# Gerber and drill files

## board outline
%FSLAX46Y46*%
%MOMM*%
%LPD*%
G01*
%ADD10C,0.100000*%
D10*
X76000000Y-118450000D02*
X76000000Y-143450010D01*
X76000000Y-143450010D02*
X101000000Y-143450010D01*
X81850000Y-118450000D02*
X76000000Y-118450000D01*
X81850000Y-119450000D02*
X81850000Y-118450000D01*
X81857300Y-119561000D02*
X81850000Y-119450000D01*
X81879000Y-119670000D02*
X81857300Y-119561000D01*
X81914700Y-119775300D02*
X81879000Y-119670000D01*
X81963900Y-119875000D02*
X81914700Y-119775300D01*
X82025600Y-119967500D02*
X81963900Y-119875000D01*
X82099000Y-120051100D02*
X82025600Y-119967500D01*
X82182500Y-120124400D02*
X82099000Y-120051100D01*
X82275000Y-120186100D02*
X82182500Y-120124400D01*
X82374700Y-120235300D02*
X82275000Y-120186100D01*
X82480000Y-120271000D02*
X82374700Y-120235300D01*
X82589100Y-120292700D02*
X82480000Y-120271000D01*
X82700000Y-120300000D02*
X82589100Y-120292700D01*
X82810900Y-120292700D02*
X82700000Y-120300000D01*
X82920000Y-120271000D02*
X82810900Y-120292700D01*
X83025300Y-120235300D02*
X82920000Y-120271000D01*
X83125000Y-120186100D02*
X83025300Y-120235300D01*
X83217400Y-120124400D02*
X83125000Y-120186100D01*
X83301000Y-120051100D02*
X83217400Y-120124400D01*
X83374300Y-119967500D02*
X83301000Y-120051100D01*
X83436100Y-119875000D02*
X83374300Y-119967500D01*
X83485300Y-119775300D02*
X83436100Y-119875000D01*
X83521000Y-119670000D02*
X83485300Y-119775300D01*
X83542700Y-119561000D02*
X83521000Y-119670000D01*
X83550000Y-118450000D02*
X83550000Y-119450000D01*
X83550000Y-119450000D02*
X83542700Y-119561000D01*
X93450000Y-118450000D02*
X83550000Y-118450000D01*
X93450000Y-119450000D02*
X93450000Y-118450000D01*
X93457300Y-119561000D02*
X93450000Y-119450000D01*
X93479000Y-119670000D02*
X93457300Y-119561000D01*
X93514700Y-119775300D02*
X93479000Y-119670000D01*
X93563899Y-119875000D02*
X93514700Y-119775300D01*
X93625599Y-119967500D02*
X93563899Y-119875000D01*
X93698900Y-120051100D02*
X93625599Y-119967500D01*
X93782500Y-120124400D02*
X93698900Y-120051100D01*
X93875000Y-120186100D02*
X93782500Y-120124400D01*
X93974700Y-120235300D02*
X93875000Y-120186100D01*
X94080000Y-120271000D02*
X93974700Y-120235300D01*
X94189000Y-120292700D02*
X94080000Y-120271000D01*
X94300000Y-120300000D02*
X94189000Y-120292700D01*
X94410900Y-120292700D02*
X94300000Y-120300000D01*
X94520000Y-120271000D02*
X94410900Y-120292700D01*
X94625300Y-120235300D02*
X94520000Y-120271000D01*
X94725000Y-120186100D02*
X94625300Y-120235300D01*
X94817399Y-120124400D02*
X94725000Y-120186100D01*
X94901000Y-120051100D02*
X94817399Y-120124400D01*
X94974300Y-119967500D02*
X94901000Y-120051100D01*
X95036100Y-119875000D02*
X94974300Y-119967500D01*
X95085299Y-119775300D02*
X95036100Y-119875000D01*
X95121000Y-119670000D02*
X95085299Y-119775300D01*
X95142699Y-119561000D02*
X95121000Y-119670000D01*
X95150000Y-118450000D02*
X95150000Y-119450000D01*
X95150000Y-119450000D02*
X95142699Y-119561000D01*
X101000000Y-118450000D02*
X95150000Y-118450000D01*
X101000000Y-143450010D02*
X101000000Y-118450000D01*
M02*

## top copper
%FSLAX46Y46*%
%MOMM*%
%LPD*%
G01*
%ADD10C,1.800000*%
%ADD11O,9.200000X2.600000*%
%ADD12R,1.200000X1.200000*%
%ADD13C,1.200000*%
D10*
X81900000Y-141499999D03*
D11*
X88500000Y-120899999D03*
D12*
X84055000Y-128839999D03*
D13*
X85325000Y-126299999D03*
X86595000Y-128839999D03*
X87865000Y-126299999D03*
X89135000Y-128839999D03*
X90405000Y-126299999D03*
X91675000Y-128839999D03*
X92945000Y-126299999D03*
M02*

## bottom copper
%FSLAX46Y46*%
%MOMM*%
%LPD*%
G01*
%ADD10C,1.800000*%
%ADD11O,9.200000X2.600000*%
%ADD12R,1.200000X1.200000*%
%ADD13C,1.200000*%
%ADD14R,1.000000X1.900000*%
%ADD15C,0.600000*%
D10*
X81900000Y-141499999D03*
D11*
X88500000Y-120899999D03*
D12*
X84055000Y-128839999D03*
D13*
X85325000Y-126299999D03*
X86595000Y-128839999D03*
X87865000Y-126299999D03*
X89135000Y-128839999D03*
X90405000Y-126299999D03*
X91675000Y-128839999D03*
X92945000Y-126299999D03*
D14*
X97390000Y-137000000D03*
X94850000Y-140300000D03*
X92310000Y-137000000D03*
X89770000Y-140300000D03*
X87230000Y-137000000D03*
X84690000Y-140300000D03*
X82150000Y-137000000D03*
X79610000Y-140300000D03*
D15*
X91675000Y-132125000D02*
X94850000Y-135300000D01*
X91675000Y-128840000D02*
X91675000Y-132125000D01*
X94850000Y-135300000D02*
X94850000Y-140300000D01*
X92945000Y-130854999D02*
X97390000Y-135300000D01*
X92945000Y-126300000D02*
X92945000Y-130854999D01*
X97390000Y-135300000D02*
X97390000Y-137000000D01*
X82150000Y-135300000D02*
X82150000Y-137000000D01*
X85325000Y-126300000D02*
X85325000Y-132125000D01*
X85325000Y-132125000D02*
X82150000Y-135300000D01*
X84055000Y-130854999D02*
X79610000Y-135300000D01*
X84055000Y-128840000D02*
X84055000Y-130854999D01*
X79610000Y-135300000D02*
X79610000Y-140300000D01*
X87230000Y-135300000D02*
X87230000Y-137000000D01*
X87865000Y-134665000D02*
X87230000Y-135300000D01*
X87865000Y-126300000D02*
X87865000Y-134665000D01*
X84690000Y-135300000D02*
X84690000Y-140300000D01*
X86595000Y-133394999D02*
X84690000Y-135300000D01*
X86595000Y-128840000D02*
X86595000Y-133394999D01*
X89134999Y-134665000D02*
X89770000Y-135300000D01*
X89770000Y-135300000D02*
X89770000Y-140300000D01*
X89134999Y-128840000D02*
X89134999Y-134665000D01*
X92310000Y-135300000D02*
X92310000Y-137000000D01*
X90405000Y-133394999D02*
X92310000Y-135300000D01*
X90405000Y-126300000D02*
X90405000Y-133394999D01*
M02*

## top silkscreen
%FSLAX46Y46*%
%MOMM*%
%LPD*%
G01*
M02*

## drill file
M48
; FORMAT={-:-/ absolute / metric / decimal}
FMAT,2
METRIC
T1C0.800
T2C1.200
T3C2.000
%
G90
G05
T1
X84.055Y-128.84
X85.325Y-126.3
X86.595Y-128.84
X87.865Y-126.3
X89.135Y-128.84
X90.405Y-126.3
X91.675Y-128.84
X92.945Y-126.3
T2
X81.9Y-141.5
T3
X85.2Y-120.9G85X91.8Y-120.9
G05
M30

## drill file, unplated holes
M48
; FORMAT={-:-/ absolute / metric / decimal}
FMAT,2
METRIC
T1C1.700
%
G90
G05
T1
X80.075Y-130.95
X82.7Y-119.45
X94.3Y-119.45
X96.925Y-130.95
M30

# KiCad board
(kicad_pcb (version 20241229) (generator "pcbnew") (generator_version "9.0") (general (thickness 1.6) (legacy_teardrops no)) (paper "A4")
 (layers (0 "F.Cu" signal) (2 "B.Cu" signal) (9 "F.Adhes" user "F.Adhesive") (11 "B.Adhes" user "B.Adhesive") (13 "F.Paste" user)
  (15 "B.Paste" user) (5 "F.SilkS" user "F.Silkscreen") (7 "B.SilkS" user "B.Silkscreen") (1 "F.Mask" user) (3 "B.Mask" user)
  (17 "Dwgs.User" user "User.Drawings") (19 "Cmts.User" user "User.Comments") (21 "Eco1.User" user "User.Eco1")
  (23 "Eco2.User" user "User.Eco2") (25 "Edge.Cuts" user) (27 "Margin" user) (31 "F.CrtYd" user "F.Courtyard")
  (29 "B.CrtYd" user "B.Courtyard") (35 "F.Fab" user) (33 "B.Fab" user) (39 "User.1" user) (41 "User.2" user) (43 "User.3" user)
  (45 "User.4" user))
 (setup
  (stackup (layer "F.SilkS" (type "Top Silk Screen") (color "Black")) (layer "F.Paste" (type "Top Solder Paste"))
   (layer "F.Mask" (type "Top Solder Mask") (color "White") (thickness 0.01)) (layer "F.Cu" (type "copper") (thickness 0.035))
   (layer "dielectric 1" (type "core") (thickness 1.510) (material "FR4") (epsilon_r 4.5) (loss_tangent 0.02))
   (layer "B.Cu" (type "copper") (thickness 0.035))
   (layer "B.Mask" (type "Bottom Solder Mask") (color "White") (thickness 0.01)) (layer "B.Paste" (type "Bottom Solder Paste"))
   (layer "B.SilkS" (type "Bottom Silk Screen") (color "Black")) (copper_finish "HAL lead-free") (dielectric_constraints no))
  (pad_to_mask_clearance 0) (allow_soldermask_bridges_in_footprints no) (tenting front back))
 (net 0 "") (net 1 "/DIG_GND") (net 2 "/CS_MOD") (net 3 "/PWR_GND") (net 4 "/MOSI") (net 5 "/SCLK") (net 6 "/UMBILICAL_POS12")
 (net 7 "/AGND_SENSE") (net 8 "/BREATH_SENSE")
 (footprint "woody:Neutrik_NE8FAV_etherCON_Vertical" (layer "F.Cu") (at 88.5 130.949999)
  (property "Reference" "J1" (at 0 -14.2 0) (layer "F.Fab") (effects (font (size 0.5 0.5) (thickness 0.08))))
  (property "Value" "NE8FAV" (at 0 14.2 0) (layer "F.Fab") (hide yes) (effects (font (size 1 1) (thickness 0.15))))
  (pad "" np_thru_hole circle (at -8.425 0) (size 1.7 1.7) (drill 1.7) (layers "*.Cu" "*.Mask"))
  (pad "" thru_hole circle (at -6.6 10.55) (size 1.8 1.8) (drill 1.2) (layers "*.Cu" "*.Mask") (remove_unused_layers no))
  (pad "" np_thru_hole circle (at -5.8 -11.5) (size 1.7 1.7) (drill 1.7) (layers "*.Cu" "*.Mask"))
  (pad "" thru_hole oval (at 0 -10.05) (size 9.2 2.6) (drill oval 8.6 2) (layers "*.Cu" "*.Mask") (remove_unused_layers no))
  (pad "" np_thru_hole circle (at 5.8 -11.5) (size 1.7 1.7) (drill 1.7) (layers "*.Cu" "*.Mask"))
  (pad "" np_thru_hole circle (at 8.425 0) (size 1.7 1.7) (drill 1.7) (layers "*.Cu" "*.Mask"))
  (pad "1" thru_hole rect (at -4.445 -2.11) (size 1.2 1.2) (drill 0.8) (layers "*.Cu" "*.Mask") (remove_unused_layers no) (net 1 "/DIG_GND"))
  (pad "2" thru_hole circle (at -3.175 -4.65) (size 1.2 1.2) (drill 0.8) (layers "*.Cu" "*.Mask") (remove_unused_layers no)
   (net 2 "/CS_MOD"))
  (pad "3" thru_hole circle (at -1.905 -2.11) (size 1.2 1.2) (drill 0.8) (layers "*.Cu" "*.Mask") (remove_unused_layers no)
   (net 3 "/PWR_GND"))
  (pad "4" thru_hole circle (at -0.635 -4.65) (size 1.2 1.2) (drill 0.8) (layers "*.Cu" "*.Mask") (remove_unused_layers no) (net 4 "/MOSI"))
  (pad "5" thru_hole circle (at 0.635 -2.11) (size 1.2 1.2) (drill 0.8) (layers "*.Cu" "*.Mask") (remove_unused_layers no) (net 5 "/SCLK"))
  (pad "6" thru_hole circle (at 1.905 -4.65) (size 1.2 1.2) (drill 0.8) (layers "*.Cu" "*.Mask") (remove_unused_layers no)
   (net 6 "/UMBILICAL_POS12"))
  (pad "7" thru_hole circle (at 3.175 -2.11) (size 1.2 1.2) (drill 0.8) (layers "*.Cu" "*.Mask") (remove_unused_layers no)
   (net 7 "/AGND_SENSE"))
  (pad "8" thru_hole circle (at 4.445 -4.65) (size 1.2 1.2) (drill 0.8) (layers "*.Cu" "*.Mask") (remove_unused_layers no)
   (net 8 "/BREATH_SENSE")))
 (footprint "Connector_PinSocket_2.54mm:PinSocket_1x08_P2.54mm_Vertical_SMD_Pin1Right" (layer "B.Cu") (at 88.5 138.65 90)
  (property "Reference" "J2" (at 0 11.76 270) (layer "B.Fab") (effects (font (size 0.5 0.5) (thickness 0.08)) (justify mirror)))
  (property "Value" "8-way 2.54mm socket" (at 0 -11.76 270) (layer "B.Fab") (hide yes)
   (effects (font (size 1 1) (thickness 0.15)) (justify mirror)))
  (pad "1" smd rect (at 1.65 8.89 90) (size 1.9 1) (layers "B.Cu" "B.Mask" "B.Paste") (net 8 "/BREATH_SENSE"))
  (pad "2" smd rect (at -1.65 6.35 90) (size 1.9 1) (layers "B.Cu" "B.Mask" "B.Paste") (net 7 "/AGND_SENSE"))
  (pad "3" smd rect (at 1.65 3.81 90) (size 1.9 1) (layers "B.Cu" "B.Mask" "B.Paste") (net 6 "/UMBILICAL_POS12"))
  (pad "4" smd rect (at -1.65 1.27 90) (size 1.9 1) (layers "B.Cu" "B.Mask" "B.Paste") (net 5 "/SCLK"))
  (pad "5" smd rect (at 1.65 -1.27 90) (size 1.9 1) (layers "B.Cu" "B.Mask" "B.Paste") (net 4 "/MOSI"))
  (pad "6" smd rect (at -1.65 -3.81 90) (size 1.9 1) (layers "B.Cu" "B.Mask" "B.Paste") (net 3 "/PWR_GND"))
  (pad "7" smd rect (at 1.65 -6.35 90) (size 1.9 1) (layers "B.Cu" "B.Mask" "B.Paste") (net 2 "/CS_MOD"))
  (pad "8" smd rect (at -1.65 -8.89 90) (size 1.9 1) (layers "B.Cu" "B.Mask" "B.Paste") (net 1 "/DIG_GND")))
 (gr_line (start 76 118.45) (end 76 143.45001) (stroke (width 0.1) (type default)) (layer "Edge.Cuts"))
 (gr_line (start 76 143.45001) (end 101 143.45001) (stroke (width 0.1) (type default)) (layer "Edge.Cuts"))
 (gr_line (start 81.85 118.45) (end 76 118.45) (stroke (width 0.1) (type default)) (layer "Edge.Cuts"))
 (gr_line (start 81.85 119.45) (end 81.85 118.45) (stroke (width 0.1) (type default)) (layer "Edge.Cuts"))
 (gr_line (start 81.8573 119.561) (end 81.85 119.45) (stroke (width 0.1) (type default)) (layer "Edge.Cuts"))
 (gr_line (start 81.879 119.67) (end 81.8573 119.561) (stroke (width 0.1) (type default)) (layer "Edge.Cuts"))
 (gr_line (start 81.9147 119.7753) (end 81.879 119.67) (stroke (width 0.1) (type default)) (layer "Edge.Cuts"))
 (gr_line (start 81.9639 119.875) (end 81.9147 119.7753) (stroke (width 0.1) (type default)) (layer "Edge.Cuts"))
 (gr_line (start 82.0256 119.9675) (end 81.9639 119.875) (stroke (width 0.1) (type default)) (layer "Edge.Cuts"))
 (gr_line (start 82.099 120.0511) (end 82.0256 119.9675) (stroke (width 0.1) (type default)) (layer "Edge.Cuts"))
 (gr_line (start 82.1825 120.1244) (end 82.099 120.0511) (stroke (width 0.1) (type default)) (layer "Edge.Cuts"))
 (gr_line (start 82.275 120.1861) (end 82.1825 120.1244) (stroke (width 0.1) (type default)) (layer "Edge.Cuts"))
 (gr_line (start 82.3747 120.2353) (end 82.275 120.1861) (stroke (width 0.1) (type default)) (layer "Edge.Cuts"))
 (gr_line (start 82.48 120.271) (end 82.3747 120.2353) (stroke (width 0.1) (type default)) (layer "Edge.Cuts"))
 (gr_line (start 82.5891 120.2927) (end 82.48 120.271) (stroke (width 0.1) (type default)) (layer "Edge.Cuts"))
 (gr_line (start 82.7 120.3) (end 82.5891 120.2927) (stroke (width 0.1) (type default)) (layer "Edge.Cuts"))
 (gr_line (start 82.8109 120.2927) (end 82.7 120.3) (stroke (width 0.1) (type default)) (layer "Edge.Cuts"))
 (gr_line (start 82.92 120.271) (end 82.8109 120.2927) (stroke (width 0.1) (type default)) (layer "Edge.Cuts"))
 (gr_line (start 83.0253 120.2353) (end 82.92 120.271) (stroke (width 0.1) (type default)) (layer "Edge.Cuts"))
 (gr_line (start 83.125 120.1861) (end 83.0253 120.2353) (stroke (width 0.1) (type default)) (layer "Edge.Cuts"))
 (gr_line (start 83.2174 120.1244) (end 83.125 120.1861) (stroke (width 0.1) (type default)) (layer "Edge.Cuts"))
 (gr_line (start 83.301 120.0511) (end 83.2174 120.1244) (stroke (width 0.1) (type default)) (layer "Edge.Cuts"))
 (gr_line (start 83.3743 119.9675) (end 83.301 120.0511) (stroke (width 0.1) (type default)) (layer "Edge.Cuts"))
 (gr_line (start 83.4361 119.875) (end 83.3743 119.9675) (stroke (width 0.1) (type default)) (layer "Edge.Cuts"))
 (gr_line (start 83.4853 119.7753) (end 83.4361 119.875) (stroke (width 0.1) (type default)) (layer "Edge.Cuts"))
 (gr_line (start 83.521 119.67) (end 83.4853 119.7753) (stroke (width 0.1) (type default)) (layer "Edge.Cuts"))
 (gr_line (start 83.5427 119.561) (end 83.521 119.67) (stroke (width 0.1) (type default)) (layer "Edge.Cuts"))
 (gr_line (start 83.55 118.45) (end 83.55 119.45) (stroke (width 0.1) (type default)) (layer "Edge.Cuts"))
 (gr_line (start 83.55 119.45) (end 83.5427 119.561) (stroke (width 0.1) (type default)) (layer "Edge.Cuts"))
 (gr_line (start 93.45 118.45) (end 83.55 118.45) (stroke (width 0.1) (type default)) (layer "Edge.Cuts"))
 (gr_line (start 93.45 119.45) (end 93.45 118.45) (stroke (width 0.1) (type default)) (layer "Edge.Cuts"))
 (gr_line (start 93.4573 119.561) (end 93.45 119.45) (stroke (width 0.1) (type default)) (layer "Edge.Cuts"))
 (gr_line (start 93.479 119.67) (end 93.4573 119.561) (stroke (width 0.1) (type default)) (layer "Edge.Cuts"))
 (gr_line (start 93.5147 119.7753) (end 93.479 119.67) (stroke (width 0.1) (type default)) (layer "Edge.Cuts"))
 (gr_line (start 93.563899 119.875) (end 93.5147 119.7753) (stroke (width 0.1) (type default)) (layer "Edge.Cuts"))
 (gr_line (start 93.625599 119.9675) (end 93.563899 119.875) (stroke (width 0.1) (type default)) (layer "Edge.Cuts"))
 (gr_line (start 93.6989 120.0511) (end 93.625599 119.9675) (stroke (width 0.1) (type default)) (layer "Edge.Cuts"))
 (gr_line (start 93.7825 120.1244) (end 93.6989 120.0511) (stroke (width 0.1) (type default)) (layer "Edge.Cuts"))
 (gr_line (start 93.875 120.1861) (end 93.7825 120.1244) (stroke (width 0.1) (type default)) (layer "Edge.Cuts"))
 (gr_line (start 93.9747 120.2353) (end 93.875 120.1861) (stroke (width 0.1) (type default)) (layer "Edge.Cuts"))
 (gr_line (start 94.08 120.271) (end 93.9747 120.2353) (stroke (width 0.1) (type default)) (layer "Edge.Cuts"))
 (gr_line (start 94.189 120.2927) (end 94.08 120.271) (stroke (width 0.1) (type default)) (layer "Edge.Cuts"))
 (gr_line (start 94.3 120.3) (end 94.189 120.2927) (stroke (width 0.1) (type default)) (layer "Edge.Cuts"))
 (gr_line (start 94.4109 120.2927) (end 94.3 120.3) (stroke (width 0.1) (type default)) (layer "Edge.Cuts"))
 (gr_line (start 94.52 120.271) (end 94.4109 120.2927) (stroke (width 0.1) (type default)) (layer "Edge.Cuts"))
 (gr_line (start 94.6253 120.2353) (end 94.52 120.271) (stroke (width 0.1) (type default)) (layer "Edge.Cuts"))
 (gr_line (start 94.725 120.1861) (end 94.6253 120.2353) (stroke (width 0.1) (type default)) (layer "Edge.Cuts"))
 (gr_line (start 94.817399 120.1244) (end 94.725 120.1861) (stroke (width 0.1) (type default)) (layer "Edge.Cuts"))
 (gr_line (start 94.901 120.0511) (end 94.817399 120.1244) (stroke (width 0.1) (type default)) (layer "Edge.Cuts"))
 (gr_line (start 94.9743 119.9675) (end 94.901 120.0511) (stroke (width 0.1) (type default)) (layer "Edge.Cuts"))
 (gr_line (start 95.0361 119.875) (end 94.9743 119.9675) (stroke (width 0.1) (type default)) (layer "Edge.Cuts"))
 (gr_line (start 95.085299 119.7753) (end 95.0361 119.875) (stroke (width 0.1) (type default)) (layer "Edge.Cuts"))
 (gr_line (start 95.121 119.67) (end 95.085299 119.7753) (stroke (width 0.1) (type default)) (layer "Edge.Cuts"))
 (gr_line (start 95.142699 119.561) (end 95.121 119.67) (stroke (width 0.1) (type default)) (layer "Edge.Cuts"))
 (gr_line (start 95.15 118.45) (end 95.15 119.45) (stroke (width 0.1) (type default)) (layer "Edge.Cuts"))
 (gr_line (start 95.15 119.45) (end 95.142699 119.561) (stroke (width 0.1) (type default)) (layer "Edge.Cuts"))
 (gr_line (start 101 118.45) (end 95.15 118.45) (stroke (width 0.1) (type default)) (layer "Edge.Cuts"))
 (gr_line (start 101 143.45001) (end 101 118.45) (stroke (width 0.1) (type default)) (layer "Edge.Cuts"))
 (segment (start 91.675 132.125) (end 94.85 135.3) (width 0.6) (layer "B.Cu") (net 7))
 (segment (start 91.675 128.84) (end 91.675 132.125) (width 0.6) (layer "B.Cu") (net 7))
 (segment (start 94.85 135.3) (end 94.85 140.3) (width 0.6) (layer "B.Cu") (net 7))
 (segment (start 92.945 130.854999) (end 97.39 135.3) (width 0.6) (layer "B.Cu") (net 8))
 (segment (start 92.945 126.3) (end 92.945 130.854999) (width 0.6) (layer "B.Cu") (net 8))
 (segment (start 97.39 135.3) (end 97.39 137) (width 0.6) (layer "B.Cu") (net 8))
 (segment (start 82.15 135.3) (end 82.15 137) (width 0.6) (layer "B.Cu") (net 2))
 (segment (start 85.325 126.3) (end 85.325 132.125) (width 0.6) (layer "B.Cu") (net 2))
 (segment (start 85.325 132.125) (end 82.15 135.3) (width 0.6) (layer "B.Cu") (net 2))
 (segment (start 84.055 130.854999) (end 79.61 135.3) (width 0.6) (layer "B.Cu") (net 1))
 (segment (start 84.055 128.84) (end 84.055 130.854999) (width 0.6) (layer "B.Cu") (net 1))
 (segment (start 79.61 135.3) (end 79.61 140.3) (width 0.6) (layer "B.Cu") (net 1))
 (segment (start 87.23 135.3) (end 87.23 137) (width 0.6) (layer "B.Cu") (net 4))
 (segment (start 87.865 134.665) (end 87.23 135.3) (width 0.6) (layer "B.Cu") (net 4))
 (segment (start 87.865 126.3) (end 87.865 134.665) (width 0.6) (layer "B.Cu") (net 4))
 (segment (start 84.69 135.3) (end 84.69 140.3) (width 0.6) (layer "B.Cu") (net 3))
 (segment (start 86.595 133.394999) (end 84.69 135.3) (width 0.6) (layer "B.Cu") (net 3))
 (segment (start 86.595 128.84) (end 86.595 133.394999) (width 0.6) (layer "B.Cu") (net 3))
 (segment (start 89.134999 134.665) (end 89.77 135.3) (width 0.6) (layer "B.Cu") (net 5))
 (segment (start 89.77 135.3) (end 89.77 140.3) (width 0.6) (layer "B.Cu") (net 5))
 (segment (start 89.134999 128.84) (end 89.134999 134.665) (width 0.6) (layer "B.Cu") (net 5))
 (segment (start 92.31 135.3) (end 92.31 137) (width 0.6) (layer "B.Cu") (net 6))
 (segment (start 90.405 133.394999) (end 92.31 135.3) (width 0.6) (layer "B.Cu") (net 6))
 (segment (start 90.405 126.3) (end 90.405 133.394999) (width 0.6) (layer "B.Cu") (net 6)))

